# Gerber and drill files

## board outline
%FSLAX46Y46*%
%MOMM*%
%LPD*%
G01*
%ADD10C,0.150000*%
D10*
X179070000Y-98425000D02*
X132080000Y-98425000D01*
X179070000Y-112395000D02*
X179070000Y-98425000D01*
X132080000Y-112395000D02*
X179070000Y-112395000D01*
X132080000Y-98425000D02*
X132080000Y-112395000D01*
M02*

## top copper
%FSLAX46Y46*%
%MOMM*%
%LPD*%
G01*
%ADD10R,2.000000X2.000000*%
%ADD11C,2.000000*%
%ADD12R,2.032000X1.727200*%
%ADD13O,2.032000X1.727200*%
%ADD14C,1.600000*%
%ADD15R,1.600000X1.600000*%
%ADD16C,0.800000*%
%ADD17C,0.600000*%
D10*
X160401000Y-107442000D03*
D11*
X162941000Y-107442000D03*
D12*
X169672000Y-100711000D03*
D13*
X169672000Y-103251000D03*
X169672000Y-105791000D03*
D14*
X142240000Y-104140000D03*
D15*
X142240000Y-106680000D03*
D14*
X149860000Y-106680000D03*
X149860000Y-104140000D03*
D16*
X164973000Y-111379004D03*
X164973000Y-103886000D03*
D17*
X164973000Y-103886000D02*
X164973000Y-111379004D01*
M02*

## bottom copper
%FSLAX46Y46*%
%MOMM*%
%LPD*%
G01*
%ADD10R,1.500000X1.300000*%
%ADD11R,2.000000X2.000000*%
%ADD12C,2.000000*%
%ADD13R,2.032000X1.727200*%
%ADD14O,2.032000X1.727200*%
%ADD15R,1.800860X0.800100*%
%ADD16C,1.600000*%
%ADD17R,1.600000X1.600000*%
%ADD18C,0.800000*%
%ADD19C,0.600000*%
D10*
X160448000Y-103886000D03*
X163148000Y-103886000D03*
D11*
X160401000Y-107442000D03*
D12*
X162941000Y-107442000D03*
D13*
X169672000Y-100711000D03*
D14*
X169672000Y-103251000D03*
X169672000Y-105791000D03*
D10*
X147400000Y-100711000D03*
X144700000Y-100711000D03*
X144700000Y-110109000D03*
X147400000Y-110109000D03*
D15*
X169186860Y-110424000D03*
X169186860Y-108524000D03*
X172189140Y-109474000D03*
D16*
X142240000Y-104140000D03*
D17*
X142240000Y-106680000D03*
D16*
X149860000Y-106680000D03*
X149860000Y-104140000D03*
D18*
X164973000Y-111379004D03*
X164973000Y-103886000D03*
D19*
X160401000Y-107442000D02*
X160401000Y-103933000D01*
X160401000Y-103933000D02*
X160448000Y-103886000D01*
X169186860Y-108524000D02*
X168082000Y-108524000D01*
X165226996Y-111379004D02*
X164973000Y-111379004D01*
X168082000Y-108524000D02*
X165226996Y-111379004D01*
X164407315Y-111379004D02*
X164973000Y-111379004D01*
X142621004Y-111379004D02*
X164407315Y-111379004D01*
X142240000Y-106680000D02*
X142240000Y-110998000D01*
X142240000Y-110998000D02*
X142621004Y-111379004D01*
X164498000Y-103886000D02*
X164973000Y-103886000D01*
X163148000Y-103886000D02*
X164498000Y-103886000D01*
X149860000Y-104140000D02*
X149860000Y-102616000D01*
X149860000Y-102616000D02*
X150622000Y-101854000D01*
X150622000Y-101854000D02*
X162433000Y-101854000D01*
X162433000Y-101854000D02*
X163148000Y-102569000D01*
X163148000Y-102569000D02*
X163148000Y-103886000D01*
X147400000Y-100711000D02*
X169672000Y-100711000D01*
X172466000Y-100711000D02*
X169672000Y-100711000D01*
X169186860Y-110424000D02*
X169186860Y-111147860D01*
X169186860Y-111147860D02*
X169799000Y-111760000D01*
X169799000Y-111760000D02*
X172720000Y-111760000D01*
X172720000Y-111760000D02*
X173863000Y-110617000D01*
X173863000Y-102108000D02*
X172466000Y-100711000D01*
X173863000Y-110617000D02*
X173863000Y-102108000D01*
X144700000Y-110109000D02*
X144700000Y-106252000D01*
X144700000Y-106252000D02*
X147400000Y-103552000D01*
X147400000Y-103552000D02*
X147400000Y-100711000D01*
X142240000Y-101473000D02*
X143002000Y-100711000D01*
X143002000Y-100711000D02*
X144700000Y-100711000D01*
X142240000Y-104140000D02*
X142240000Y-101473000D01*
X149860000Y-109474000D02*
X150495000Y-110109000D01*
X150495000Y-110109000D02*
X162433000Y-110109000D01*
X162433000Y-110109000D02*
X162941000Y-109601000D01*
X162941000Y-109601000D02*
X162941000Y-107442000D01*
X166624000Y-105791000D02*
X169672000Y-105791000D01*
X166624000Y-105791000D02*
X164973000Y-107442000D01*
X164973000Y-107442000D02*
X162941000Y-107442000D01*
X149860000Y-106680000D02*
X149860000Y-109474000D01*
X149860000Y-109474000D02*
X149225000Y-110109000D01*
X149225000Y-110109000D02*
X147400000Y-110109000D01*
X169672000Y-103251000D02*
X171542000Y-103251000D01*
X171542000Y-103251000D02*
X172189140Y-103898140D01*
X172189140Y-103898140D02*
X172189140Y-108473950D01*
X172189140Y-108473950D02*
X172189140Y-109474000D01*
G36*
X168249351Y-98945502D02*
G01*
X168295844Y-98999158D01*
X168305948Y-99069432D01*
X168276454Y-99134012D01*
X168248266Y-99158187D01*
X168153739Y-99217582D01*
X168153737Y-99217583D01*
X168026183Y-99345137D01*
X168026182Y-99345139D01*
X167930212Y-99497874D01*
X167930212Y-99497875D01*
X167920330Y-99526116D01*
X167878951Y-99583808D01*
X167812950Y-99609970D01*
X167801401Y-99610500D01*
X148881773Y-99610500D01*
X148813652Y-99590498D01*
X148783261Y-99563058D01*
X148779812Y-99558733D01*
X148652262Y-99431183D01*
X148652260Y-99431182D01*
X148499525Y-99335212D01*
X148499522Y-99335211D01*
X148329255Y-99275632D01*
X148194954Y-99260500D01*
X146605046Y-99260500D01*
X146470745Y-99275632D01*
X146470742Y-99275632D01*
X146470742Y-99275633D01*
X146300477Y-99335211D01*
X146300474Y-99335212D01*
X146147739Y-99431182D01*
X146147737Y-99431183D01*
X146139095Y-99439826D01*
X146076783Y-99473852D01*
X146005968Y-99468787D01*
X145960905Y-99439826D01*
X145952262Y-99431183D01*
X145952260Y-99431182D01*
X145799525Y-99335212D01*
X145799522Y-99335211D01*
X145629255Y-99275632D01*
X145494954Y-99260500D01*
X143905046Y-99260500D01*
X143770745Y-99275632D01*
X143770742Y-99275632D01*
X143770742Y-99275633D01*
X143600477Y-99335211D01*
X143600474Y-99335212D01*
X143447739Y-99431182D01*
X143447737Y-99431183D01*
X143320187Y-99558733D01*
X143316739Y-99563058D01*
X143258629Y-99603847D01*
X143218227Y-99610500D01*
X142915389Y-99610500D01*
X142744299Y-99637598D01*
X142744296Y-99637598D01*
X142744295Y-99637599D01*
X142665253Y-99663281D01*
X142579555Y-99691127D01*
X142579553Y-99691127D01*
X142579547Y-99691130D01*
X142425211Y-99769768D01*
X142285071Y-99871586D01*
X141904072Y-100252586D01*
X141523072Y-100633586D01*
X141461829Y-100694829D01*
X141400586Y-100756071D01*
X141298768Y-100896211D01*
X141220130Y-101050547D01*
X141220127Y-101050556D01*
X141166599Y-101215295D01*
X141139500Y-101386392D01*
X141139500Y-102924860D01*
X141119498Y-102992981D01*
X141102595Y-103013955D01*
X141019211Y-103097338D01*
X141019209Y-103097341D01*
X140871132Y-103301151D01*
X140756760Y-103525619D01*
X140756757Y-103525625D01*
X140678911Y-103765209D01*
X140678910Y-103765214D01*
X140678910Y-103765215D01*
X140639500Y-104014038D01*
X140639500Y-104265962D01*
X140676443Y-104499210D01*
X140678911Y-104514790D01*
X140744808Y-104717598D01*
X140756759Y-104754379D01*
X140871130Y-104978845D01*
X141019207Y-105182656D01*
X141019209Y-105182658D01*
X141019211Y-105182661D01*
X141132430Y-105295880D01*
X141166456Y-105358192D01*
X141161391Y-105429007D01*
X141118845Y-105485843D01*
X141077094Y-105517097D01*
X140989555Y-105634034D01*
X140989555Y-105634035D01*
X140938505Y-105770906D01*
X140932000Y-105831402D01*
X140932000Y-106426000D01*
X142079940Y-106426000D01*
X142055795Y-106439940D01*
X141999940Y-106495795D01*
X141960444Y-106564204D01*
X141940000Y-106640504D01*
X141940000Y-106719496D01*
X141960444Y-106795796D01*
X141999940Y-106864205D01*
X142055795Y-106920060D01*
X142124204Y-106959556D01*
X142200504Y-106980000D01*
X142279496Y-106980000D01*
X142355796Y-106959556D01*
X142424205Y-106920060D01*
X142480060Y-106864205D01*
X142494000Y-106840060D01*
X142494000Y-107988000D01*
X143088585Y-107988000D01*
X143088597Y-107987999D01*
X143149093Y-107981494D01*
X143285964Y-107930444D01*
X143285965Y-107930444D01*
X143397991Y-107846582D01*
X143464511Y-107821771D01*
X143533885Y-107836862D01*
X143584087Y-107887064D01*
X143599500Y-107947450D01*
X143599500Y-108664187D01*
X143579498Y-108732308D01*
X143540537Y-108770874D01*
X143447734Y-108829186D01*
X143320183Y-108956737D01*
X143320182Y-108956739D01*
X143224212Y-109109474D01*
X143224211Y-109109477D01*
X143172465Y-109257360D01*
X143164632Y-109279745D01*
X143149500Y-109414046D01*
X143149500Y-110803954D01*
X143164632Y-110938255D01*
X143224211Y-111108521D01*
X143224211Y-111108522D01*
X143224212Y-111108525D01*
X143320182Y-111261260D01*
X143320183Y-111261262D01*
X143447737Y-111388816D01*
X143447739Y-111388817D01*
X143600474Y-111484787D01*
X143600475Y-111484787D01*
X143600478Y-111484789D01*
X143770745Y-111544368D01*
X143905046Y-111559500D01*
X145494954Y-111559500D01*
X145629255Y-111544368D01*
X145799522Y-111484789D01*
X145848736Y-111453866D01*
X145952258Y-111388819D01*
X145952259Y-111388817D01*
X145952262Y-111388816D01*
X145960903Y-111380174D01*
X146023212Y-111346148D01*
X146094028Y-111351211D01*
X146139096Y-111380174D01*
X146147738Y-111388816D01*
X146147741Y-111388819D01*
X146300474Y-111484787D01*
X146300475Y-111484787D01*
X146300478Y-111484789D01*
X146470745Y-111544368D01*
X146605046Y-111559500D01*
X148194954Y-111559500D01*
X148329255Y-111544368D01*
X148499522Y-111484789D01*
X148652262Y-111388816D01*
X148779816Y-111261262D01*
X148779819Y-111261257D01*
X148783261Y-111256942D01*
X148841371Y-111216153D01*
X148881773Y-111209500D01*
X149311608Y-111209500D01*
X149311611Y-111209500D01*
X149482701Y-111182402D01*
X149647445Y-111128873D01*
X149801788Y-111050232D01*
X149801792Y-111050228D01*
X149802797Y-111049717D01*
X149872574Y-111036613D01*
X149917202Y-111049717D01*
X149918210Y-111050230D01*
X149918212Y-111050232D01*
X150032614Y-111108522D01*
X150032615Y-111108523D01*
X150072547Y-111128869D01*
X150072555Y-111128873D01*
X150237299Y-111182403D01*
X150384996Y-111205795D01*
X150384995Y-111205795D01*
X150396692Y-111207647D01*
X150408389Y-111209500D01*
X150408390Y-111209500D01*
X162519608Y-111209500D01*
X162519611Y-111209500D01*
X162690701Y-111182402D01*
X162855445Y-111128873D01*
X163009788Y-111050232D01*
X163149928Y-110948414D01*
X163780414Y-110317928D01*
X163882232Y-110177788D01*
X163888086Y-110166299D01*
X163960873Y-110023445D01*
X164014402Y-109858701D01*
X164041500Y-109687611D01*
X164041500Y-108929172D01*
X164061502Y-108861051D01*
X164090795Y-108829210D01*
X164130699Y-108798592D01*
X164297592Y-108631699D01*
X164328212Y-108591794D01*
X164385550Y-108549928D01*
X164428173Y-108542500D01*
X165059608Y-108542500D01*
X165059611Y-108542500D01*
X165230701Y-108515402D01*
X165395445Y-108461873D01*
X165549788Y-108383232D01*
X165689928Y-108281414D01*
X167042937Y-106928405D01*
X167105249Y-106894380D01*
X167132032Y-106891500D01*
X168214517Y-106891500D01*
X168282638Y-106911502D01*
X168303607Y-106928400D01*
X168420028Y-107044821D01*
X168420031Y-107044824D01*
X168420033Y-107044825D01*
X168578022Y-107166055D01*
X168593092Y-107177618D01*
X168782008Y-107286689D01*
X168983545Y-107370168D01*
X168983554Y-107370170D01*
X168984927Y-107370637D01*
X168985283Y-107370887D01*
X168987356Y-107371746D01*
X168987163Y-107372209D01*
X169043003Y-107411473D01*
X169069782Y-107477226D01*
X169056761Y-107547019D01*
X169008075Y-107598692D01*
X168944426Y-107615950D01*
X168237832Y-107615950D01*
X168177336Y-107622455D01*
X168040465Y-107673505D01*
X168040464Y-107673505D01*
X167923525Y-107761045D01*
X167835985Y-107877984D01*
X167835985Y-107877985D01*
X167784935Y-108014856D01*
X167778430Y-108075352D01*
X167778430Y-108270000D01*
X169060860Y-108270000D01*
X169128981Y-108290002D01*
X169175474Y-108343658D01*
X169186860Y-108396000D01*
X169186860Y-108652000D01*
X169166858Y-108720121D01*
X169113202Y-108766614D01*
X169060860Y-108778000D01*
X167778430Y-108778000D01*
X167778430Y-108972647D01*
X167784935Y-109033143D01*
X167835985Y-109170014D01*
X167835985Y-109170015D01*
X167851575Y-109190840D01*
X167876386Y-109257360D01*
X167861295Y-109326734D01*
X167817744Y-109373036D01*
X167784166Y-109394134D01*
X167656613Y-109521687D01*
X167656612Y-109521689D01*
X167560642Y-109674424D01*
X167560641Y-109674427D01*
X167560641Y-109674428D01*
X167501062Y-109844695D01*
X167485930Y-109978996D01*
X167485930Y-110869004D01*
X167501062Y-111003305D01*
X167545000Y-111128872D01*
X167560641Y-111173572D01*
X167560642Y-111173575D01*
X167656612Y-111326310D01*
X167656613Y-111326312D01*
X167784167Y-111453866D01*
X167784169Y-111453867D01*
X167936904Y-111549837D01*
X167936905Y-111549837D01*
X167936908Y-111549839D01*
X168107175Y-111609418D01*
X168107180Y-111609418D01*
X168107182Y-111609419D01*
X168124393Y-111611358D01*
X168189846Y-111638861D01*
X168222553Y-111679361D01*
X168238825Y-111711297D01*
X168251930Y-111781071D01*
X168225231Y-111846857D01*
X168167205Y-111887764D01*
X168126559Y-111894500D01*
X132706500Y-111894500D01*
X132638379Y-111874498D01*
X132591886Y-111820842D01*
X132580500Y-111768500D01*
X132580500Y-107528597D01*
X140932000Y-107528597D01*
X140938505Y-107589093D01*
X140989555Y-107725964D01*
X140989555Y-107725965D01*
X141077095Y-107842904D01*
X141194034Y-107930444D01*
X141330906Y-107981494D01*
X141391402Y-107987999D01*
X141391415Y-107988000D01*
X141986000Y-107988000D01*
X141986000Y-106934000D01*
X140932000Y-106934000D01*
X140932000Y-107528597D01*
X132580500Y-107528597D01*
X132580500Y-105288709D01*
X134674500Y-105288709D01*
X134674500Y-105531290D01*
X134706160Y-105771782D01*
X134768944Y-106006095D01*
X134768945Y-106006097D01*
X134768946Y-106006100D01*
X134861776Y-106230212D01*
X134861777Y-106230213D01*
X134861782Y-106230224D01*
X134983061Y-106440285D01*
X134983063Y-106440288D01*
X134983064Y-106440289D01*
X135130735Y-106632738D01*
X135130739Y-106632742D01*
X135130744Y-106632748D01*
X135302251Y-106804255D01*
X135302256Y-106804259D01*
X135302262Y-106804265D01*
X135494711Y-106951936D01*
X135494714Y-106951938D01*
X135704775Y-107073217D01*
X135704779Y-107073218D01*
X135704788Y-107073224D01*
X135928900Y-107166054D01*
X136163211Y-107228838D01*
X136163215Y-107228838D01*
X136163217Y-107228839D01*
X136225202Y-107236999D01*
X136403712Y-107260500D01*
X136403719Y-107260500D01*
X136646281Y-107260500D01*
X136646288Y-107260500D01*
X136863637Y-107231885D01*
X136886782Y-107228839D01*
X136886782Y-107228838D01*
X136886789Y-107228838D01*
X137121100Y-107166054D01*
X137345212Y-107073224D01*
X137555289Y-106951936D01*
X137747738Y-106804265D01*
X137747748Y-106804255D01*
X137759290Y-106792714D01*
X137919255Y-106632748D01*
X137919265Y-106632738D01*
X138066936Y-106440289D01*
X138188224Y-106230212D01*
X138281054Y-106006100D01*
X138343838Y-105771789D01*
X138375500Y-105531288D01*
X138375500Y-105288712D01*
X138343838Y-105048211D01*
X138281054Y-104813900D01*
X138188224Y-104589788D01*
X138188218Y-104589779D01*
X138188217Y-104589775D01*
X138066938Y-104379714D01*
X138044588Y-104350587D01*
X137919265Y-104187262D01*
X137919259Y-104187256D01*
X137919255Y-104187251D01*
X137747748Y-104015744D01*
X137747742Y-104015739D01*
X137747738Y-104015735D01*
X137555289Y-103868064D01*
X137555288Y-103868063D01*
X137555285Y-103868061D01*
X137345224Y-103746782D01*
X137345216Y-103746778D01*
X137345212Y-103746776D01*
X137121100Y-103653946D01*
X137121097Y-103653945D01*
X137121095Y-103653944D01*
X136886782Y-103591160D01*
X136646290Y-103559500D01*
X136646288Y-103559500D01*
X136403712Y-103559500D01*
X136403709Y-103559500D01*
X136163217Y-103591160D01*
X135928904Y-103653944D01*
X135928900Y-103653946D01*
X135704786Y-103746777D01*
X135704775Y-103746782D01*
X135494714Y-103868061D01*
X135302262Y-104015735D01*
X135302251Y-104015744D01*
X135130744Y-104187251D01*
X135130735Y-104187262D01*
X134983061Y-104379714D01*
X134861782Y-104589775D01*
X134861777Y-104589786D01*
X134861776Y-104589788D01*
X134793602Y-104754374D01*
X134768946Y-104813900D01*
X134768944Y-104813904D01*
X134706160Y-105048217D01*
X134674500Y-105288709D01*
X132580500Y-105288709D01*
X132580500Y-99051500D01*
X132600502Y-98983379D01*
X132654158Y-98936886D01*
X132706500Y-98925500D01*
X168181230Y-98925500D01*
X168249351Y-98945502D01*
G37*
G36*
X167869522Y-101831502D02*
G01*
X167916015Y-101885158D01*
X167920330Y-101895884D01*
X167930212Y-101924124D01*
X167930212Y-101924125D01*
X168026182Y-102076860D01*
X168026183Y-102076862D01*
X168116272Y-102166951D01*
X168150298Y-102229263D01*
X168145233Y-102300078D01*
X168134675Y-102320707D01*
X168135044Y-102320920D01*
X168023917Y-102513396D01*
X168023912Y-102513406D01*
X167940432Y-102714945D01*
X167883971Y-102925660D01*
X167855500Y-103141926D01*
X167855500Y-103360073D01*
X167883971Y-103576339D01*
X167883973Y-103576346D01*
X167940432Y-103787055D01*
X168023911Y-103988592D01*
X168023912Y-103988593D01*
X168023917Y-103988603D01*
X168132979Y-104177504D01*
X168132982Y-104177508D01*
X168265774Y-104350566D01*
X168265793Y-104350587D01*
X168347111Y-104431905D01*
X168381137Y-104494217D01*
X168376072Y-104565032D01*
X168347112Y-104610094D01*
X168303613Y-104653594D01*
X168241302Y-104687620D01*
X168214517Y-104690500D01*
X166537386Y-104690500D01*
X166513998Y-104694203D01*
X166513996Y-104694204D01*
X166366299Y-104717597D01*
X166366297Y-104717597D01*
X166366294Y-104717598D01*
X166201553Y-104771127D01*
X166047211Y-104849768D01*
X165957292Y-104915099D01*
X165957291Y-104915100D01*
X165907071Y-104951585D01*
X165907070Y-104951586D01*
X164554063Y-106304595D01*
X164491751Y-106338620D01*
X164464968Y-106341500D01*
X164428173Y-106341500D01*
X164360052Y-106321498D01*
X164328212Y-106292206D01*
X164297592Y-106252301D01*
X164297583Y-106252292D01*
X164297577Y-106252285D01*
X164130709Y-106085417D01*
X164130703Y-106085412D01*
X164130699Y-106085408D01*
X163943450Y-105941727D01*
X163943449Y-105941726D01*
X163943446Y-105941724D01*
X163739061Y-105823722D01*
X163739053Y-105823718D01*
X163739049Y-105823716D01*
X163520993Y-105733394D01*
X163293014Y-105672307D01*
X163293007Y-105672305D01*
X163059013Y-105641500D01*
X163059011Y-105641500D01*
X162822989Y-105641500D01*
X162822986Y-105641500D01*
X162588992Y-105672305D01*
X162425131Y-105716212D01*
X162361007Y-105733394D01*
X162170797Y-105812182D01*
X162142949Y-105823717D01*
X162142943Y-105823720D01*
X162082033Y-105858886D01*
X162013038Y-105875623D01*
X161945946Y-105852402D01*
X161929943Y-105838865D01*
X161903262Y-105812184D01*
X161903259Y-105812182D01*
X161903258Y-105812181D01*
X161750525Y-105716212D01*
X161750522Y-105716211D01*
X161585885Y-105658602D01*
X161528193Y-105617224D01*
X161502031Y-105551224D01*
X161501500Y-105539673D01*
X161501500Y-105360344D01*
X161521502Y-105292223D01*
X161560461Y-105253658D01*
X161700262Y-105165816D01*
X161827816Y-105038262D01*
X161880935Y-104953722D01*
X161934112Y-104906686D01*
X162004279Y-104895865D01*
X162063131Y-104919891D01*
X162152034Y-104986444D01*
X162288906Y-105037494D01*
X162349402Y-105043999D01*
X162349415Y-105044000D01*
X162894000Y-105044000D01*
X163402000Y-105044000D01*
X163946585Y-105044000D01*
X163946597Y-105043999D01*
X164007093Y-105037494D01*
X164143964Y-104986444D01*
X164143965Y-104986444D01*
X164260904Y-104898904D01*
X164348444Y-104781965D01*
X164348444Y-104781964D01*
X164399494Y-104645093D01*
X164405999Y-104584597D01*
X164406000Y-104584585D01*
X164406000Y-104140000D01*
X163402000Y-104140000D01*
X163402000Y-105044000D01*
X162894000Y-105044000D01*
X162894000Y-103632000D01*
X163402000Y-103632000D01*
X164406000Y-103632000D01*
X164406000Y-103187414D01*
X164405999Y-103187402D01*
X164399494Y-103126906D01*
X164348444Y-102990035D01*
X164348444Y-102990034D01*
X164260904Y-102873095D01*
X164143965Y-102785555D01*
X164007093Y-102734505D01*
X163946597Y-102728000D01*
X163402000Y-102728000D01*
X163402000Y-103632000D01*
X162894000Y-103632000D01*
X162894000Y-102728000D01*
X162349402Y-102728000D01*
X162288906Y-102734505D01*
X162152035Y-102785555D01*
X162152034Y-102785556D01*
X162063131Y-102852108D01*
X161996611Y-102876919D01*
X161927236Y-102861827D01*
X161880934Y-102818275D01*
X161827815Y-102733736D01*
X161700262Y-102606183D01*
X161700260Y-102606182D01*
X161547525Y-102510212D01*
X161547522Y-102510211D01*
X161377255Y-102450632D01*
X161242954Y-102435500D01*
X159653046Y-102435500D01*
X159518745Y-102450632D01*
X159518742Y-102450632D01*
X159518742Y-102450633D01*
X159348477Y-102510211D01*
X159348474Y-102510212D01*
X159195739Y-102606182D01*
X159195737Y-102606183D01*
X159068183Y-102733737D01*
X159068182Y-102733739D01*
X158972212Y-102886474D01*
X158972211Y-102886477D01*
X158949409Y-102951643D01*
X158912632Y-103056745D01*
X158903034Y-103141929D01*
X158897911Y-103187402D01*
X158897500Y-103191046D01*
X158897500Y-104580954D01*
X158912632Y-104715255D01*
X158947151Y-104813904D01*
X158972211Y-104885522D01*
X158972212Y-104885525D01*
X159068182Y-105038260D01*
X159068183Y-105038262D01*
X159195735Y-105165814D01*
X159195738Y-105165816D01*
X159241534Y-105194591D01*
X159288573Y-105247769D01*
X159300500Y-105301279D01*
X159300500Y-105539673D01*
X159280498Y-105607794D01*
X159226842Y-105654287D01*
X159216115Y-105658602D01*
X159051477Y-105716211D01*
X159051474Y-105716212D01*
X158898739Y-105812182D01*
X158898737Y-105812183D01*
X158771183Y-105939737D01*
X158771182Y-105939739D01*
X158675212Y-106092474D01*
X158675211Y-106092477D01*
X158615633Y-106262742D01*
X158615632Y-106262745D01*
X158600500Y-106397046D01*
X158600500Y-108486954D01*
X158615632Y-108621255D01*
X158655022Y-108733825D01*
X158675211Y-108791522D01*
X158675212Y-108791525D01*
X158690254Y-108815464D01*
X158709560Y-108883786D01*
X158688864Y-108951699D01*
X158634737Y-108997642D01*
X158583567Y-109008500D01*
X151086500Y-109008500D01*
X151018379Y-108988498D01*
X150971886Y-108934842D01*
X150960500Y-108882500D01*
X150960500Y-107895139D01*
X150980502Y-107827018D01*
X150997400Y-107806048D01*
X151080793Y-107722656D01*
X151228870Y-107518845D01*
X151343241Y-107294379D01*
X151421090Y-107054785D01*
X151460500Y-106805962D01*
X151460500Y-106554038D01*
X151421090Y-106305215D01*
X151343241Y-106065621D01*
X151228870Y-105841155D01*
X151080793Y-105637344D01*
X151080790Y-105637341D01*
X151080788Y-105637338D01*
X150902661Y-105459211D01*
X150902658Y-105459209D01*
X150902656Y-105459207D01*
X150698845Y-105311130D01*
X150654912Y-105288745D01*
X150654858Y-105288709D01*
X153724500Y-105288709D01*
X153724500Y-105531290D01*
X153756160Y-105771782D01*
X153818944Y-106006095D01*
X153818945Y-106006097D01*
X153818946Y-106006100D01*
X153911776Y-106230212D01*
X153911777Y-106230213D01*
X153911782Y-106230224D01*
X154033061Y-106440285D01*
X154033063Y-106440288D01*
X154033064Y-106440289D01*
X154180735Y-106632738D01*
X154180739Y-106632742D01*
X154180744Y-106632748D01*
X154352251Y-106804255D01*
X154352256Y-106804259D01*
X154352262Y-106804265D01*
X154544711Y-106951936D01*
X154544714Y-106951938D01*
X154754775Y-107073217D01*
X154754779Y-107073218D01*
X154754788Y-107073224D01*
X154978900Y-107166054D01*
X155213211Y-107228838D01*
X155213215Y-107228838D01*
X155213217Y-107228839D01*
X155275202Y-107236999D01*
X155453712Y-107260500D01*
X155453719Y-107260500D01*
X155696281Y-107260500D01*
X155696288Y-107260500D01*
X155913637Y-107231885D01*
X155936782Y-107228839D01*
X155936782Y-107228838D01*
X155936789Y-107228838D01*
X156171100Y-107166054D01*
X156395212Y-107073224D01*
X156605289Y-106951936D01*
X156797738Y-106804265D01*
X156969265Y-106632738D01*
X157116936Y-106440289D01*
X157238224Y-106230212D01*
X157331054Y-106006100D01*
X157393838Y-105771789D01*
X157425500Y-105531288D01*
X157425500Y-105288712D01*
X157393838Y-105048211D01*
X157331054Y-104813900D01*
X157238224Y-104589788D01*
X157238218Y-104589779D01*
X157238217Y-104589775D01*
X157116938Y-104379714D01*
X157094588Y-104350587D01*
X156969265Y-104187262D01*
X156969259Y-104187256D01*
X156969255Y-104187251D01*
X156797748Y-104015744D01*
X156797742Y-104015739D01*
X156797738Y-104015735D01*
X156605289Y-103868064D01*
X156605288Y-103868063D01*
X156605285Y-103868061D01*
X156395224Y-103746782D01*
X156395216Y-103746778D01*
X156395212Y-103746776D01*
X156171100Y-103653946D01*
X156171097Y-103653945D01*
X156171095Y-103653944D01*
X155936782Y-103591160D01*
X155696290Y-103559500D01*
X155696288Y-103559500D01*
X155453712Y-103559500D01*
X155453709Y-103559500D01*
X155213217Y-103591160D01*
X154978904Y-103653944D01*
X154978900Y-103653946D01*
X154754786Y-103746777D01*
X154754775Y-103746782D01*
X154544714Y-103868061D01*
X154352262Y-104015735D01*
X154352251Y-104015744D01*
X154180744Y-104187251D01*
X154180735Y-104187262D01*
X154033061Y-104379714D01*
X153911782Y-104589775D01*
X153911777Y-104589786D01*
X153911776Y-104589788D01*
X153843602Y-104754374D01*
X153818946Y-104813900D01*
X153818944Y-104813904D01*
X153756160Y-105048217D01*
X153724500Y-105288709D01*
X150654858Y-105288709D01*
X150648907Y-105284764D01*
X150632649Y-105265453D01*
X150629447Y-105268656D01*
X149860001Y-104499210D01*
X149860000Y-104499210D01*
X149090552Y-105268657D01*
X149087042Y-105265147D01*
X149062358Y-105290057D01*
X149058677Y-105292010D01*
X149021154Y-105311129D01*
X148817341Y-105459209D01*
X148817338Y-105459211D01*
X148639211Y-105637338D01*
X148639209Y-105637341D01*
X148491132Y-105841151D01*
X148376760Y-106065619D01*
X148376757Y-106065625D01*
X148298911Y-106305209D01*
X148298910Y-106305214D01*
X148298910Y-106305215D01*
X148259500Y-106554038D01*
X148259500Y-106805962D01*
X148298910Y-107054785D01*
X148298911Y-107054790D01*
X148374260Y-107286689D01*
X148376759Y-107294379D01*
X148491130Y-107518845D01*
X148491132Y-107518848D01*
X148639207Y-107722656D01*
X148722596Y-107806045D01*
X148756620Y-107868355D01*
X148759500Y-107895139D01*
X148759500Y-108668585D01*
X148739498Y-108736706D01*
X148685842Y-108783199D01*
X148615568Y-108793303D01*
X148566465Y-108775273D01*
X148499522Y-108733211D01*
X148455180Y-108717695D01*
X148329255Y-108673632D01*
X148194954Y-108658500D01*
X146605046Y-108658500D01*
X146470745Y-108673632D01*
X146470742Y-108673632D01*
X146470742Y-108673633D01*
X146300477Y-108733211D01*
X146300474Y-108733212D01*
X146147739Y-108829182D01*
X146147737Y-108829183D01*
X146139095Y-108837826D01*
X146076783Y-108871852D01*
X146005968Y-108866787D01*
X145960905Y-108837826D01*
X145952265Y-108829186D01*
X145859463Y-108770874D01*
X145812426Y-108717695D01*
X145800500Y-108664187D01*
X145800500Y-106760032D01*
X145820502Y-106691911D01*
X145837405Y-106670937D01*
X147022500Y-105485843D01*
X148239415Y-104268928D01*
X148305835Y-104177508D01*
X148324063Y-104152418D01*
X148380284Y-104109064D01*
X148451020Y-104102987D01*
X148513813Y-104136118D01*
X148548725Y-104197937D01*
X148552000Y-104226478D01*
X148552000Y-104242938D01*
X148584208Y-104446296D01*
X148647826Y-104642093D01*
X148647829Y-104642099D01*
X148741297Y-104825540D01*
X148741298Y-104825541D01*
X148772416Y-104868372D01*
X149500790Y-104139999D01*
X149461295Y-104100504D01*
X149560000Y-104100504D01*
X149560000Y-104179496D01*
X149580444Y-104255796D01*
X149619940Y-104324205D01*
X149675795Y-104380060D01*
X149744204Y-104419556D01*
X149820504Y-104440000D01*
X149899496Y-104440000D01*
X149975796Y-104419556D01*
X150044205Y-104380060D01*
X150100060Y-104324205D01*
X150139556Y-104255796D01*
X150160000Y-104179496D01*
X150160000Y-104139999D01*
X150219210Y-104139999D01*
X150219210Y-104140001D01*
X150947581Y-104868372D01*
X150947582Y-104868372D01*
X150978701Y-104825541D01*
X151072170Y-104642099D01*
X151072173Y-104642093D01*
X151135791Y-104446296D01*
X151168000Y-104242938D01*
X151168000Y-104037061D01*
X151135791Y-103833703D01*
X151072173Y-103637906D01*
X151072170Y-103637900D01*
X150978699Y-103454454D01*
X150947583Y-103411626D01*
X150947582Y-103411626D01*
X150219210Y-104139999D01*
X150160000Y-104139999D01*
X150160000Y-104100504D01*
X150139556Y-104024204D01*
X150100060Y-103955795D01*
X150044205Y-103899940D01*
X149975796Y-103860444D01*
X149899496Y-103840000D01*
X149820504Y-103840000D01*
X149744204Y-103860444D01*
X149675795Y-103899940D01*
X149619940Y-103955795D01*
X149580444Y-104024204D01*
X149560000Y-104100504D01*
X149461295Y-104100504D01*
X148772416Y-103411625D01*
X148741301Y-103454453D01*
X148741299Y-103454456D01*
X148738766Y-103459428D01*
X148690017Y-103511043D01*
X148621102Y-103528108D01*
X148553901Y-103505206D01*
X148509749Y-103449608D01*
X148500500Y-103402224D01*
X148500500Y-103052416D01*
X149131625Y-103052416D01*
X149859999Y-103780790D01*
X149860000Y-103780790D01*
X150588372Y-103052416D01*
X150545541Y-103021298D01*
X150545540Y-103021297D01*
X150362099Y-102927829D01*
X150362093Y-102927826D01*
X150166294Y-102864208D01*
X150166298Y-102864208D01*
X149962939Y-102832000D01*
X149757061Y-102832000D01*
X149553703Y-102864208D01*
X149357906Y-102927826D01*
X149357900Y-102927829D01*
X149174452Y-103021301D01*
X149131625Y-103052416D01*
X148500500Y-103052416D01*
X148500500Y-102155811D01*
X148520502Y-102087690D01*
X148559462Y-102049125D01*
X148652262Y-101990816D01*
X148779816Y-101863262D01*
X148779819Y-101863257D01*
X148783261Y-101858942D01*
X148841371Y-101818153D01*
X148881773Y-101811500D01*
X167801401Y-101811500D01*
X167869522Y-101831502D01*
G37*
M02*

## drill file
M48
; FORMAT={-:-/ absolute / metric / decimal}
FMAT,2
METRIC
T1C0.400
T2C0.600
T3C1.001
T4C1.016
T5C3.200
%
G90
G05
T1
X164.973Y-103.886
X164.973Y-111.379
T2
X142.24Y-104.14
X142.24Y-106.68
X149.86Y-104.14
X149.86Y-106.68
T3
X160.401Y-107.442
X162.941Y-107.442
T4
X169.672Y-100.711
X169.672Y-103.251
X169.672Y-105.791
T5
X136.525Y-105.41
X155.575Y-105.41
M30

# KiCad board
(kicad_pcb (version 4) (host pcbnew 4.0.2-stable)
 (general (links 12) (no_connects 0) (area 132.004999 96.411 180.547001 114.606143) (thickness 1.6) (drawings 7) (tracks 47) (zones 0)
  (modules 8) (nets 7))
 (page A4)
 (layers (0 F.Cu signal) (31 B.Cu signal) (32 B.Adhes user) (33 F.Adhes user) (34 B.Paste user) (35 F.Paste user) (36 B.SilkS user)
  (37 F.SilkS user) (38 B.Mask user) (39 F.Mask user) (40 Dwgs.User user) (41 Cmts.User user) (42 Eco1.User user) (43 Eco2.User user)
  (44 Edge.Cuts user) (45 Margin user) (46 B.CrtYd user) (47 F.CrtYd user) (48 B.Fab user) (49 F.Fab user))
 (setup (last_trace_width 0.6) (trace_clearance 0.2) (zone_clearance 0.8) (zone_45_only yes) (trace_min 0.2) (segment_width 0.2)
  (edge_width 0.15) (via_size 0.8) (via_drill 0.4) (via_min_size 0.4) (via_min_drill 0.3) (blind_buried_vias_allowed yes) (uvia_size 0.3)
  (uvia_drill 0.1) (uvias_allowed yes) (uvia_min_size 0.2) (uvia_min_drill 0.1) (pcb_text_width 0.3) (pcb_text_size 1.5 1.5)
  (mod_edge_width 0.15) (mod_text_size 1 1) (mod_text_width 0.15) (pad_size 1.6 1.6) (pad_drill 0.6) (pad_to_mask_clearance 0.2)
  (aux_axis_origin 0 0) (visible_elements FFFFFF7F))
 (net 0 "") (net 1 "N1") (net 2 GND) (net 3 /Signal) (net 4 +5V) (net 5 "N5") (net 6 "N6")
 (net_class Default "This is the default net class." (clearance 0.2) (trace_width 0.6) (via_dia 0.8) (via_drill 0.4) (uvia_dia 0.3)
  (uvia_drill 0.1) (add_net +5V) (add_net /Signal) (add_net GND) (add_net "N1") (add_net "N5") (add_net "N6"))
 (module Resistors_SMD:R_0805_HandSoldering (layer B.Cu) (at 161.798 103.886)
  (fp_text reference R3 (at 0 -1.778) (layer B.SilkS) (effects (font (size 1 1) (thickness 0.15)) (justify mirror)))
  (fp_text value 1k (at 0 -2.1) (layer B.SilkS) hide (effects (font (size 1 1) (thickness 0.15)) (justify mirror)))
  (pad 1 smd rect (at -1.35 0) (size 1.5 1.3) (layers B.Cu B.Paste B.Mask) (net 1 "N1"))
  (pad 2 smd rect (at 1.35 0) (size 1.5 1.3) (layers B.Cu B.Paste B.Mask) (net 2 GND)))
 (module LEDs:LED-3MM (layer F.Cu) (at 160.401 107.442)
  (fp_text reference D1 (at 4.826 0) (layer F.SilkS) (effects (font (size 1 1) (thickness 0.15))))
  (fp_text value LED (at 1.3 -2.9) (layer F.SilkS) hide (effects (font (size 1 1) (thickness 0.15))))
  (pad 1 thru_hole rect (at 0 0 90) (size 2 2) (drill 1.00076) (layers *.Cu *.Mask F.SilkS) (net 1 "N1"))
  (pad 2 thru_hole circle (at 2.54 0) (size 2 2) (drill 1.00076) (layers *.Cu *.Mask F.SilkS) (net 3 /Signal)))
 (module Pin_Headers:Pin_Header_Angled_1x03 (layer F.Cu) (at 169.672 100.711)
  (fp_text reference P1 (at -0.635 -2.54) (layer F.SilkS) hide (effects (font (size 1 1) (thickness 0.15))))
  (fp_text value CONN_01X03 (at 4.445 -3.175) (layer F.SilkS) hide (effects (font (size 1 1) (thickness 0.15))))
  (pad 1 thru_hole rect (at 0 0) (size 2.032 1.7272) (drill 1.016) (layers *.Cu *.Mask F.SilkS) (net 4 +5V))
  (pad 2 thru_hole oval (at 0 2.54) (size 2.032 1.7272) (drill 1.016) (layers *.Cu *.Mask F.SilkS) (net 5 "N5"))
  (pad 3 thru_hole oval (at 0 5.08) (size 2.032 1.7272) (drill 1.016) (layers *.Cu *.Mask F.SilkS) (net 3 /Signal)))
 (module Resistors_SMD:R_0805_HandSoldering (layer B.Cu) (at 146.05 100.711 180)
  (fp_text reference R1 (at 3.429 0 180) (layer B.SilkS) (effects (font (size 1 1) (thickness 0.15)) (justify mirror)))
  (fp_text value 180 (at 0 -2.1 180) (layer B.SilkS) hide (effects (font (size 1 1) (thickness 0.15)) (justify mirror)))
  (pad 1 smd rect (at -1.35 0 180) (size 1.5 1.3) (layers B.Cu B.Paste B.Mask) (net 4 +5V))
  (pad 2 smd rect (at 1.35 0 180) (size 1.5 1.3) (layers B.Cu B.Paste B.Mask) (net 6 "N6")))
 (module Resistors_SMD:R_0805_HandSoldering (layer B.Cu) (at 146.05 110.109)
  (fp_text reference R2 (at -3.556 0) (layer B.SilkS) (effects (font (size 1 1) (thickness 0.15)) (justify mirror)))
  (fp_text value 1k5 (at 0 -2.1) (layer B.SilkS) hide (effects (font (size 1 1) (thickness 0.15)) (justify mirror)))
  (pad 1 smd rect (at -1.35 0) (size 1.5 1.3) (layers B.Cu B.Paste B.Mask) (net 4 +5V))
  (pad 2 smd rect (at 1.35 0) (size 1.5 1.3) (layers B.Cu B.Paste B.Mask) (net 3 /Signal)))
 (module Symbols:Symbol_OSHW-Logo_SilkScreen (layer B.Cu) (at 175.133 102.235 180)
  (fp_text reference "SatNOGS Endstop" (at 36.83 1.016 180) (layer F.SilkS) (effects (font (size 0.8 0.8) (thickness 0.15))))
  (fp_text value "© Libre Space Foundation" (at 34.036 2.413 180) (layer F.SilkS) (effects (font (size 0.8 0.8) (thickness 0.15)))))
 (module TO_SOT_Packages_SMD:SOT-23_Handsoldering (layer B.Cu) (at 170.688 109.474 90)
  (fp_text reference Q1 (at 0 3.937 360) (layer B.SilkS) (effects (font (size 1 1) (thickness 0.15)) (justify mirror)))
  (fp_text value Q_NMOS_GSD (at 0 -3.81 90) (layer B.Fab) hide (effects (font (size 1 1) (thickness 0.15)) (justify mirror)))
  (pad 1 smd rect (at -0.95 -1.50114 90) (size 0.8001 1.80086) (layers B.Cu B.Paste B.Mask) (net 4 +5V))
  (pad 2 smd rect (at 0.95 -1.50114 90) (size 0.8001 1.80086) (layers B.Cu B.Paste B.Mask) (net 2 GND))
  (pad 3 smd rect (at 0 1.50114 90) (size 0.8001 1.80086) (layers B.Cu B.Paste B.Mask) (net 5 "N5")))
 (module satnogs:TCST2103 (layer F.Cu) (at 146.05 105.41)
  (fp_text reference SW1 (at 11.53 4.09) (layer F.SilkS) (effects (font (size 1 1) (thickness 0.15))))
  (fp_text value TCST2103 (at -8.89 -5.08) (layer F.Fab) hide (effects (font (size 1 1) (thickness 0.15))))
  (pad 1 thru_hole circle (at -3.81 -1.27) (size 1.6 1.6) (drill 0.6) (layers *.Cu *.Mask F.SilkS) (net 6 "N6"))
  (pad 2 thru_hole rect (at -3.81 1.27) (size 1.6 1.6) (drill 0.6) (layers *.Cu *.Mask F.SilkS) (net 2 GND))
  (pad 3 thru_hole circle (at 3.81 1.27) (size 1.6 1.6) (drill 0.6) (layers *.Cu *.Mask F.SilkS) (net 3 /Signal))
  (pad 4 thru_hole circle (at 3.81 -1.27) (size 1.6 1.6) (drill 0.6) (layers *.Cu *.Mask F.SilkS) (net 2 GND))
  (pad "" np_thru_hole circle (at 9.525 0) (size 3.2 3.2) (drill 3.2) (layers *.Cu *.Mask F.SilkS))
  (pad "" np_thru_hole circle (at -9.525 0) (size 3.2 3.2) (drill 3.2) (layers *.Cu *.Mask F.SilkS)))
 (gr_line (start 179.07 98.425) (end 132.08 98.425) (angle 90) (layer Edge.Cuts) (width 0.15))
 (gr_line (start 179.07 112.395) (end 179.07 98.425) (angle 90) (layer Edge.Cuts) (width 0.15))
 (gr_line (start 132.08 112.395) (end 179.07 112.395) (angle 90) (layer Edge.Cuts) (width 0.15))
 (gr_line (start 132.08 98.425) (end 132.08 112.395) (angle 90) (layer Edge.Cuts) (width 0.15))
 (segment (start 160.401 107.442) (end 160.401 103.933) (width 0.6) (layer B.Cu) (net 1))
 (segment (start 160.401 103.933) (end 160.448 103.886) (width 0.6) (layer B.Cu) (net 1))
 (segment (start 169.18686 108.524) (end 168.082 108.524) (width 0.6) (layer B.Cu) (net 2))
 (segment (start 165.226996 111.379004) (end 164.973 111.379004) (width 0.6) (layer B.Cu) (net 2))
 (segment (start 168.082 108.524) (end 165.226996 111.379004) (width 0.6) (layer B.Cu) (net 2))
 (segment (start 164.407315 111.379004) (end 164.973 111.379004) (width 0.6) (layer B.Cu) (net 2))
 (segment (start 142.621004 111.379004) (end 164.407315 111.379004) (width 0.6) (layer B.Cu) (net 2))
 (segment (start 142.24 106.68) (end 142.24 110.998) (width 0.6) (layer B.Cu) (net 2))
 (via (at 164.973 111.379004) (size 0.8) (drill 0.4) (layers F.Cu B.Cu) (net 2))
 (segment (start 142.24 110.998) (end 142.621004 111.379004) (width 0.6) (layer B.Cu) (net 2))
 (segment (start 164.973 103.886) (end 164.973 111.379004) (width 0.6) (layer F.Cu) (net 2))
 (segment (start 164.498 103.886) (end 164.973 103.886) (width 0.6) (layer B.Cu) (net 2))
 (via (at 164.973 103.886) (size 0.8) (drill 0.4) (layers F.Cu B.Cu) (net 2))
 (segment (start 163.148 103.886) (end 164.498 103.886) (width 0.6) (layer B.Cu) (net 2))
 (segment (start 149.86 104.14) (end 149.86 102.616) (width 0.6) (layer B.Cu) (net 2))
 (segment (start 149.86 102.616) (end 150.622 101.854) (width 0.6) (layer B.Cu) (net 2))
 (segment (start 150.622 101.854) (end 162.433 101.854) (width 0.6) (layer B.Cu) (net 2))
 (segment (start 162.433 101.854) (end 163.148 102.569) (width 0.6) (layer B.Cu) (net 2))
 (segment (start 163.148 102.569) (end 163.148 103.886) (width 0.6) (layer B.Cu) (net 2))
 (segment (start 147.4 100.711) (end 169.672 100.711) (width 0.6) (layer B.Cu) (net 4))
 (segment (start 172.466 100.711) (end 169.672 100.711) (width 0.6) (layer B.Cu) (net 4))
 (segment (start 169.18686 110.424) (end 169.18686 111.14786) (width 0.6) (layer B.Cu) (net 4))
 (segment (start 169.18686 111.14786) (end 169.799 111.76) (width 0.6) (layer B.Cu) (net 4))
 (segment (start 169.799 111.76) (end 172.72 111.76) (width 0.6) (layer B.Cu) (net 4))
 (segment (start 172.72 111.76) (end 173.863 110.617) (width 0.6) (layer B.Cu) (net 4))
 (segment (start 173.863 102.108) (end 172.466 100.711) (width 0.6) (layer B.Cu) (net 4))
 (segment (start 173.863 110.617) (end 173.863 102.108) (width 0.6) (layer B.Cu) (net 4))
 (segment (start 144.7 110.109) (end 144.7 106.252) (width 0.6) (layer B.Cu) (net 4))
 (segment (start 144.7 106.252) (end 147.4 103.552) (width 0.6) (layer B.Cu) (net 4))
 (segment (start 147.4 103.552) (end 147.4 100.711) (width 0.6) (layer B.Cu) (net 4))
 (segment (start 142.24 101.473) (end 143.002 100.711) (width 0.6) (layer B.Cu) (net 6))
 (segment (start 143.002 100.711) (end 144.7 100.711) (width 0.6) (layer B.Cu) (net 6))
 (segment (start 142.24 104.14) (end 142.24 101.473) (width 0.6) (layer B.Cu) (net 6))
 (segment (start 149.86 109.474) (end 150.495 110.109) (width 0.6) (layer B.Cu) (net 3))
 (segment (start 150.495 110.109) (end 162.433 110.109) (width 0.6) (layer B.Cu) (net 3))
 (segment (start 162.433 110.109) (end 162.941 109.601) (width 0.6) (layer B.Cu) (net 3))
 (segment (start 162.941 109.601) (end 162.941 107.442) (width 0.6) (layer B.Cu) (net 3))
 (segment (start 166.624 105.791) (end 169.672 105.791) (width 0.6) (layer B.Cu) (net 3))
 (segment (start 166.624 105.791) (end 164.973 107.442) (width 0.6) (layer B.Cu) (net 3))
 (segment (start 164.973 107.442) (end 162.941 107.442) (width 0.6) (layer B.Cu) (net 3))
 (segment (start 149.86 106.68) (end 149.86 109.474) (width 0.6) (layer B.Cu) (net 3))
 (segment (start 149.86 109.474) (end 149.225 110.109) (width 0.6) (layer B.Cu) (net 3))
 (segment (start 149.225 110.109) (end 147.4 110.109) (width 0.6) (layer B.Cu) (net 3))
 (segment (start 169.672 103.251) (end 171.542 103.251) (width 0.6) (layer B.Cu) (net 5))
 (segment (start 171.542 103.251) (end 172.18914 103.89814) (width 0.6) (layer B.Cu) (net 5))
 (segment (start 172.18914 103.89814) (end 172.18914 108.47395) (width 0.6) (layer B.Cu) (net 5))
 (segment (start 172.18914 108.47395) (end 172.18914 109.474) (width 0.6) (layer B.Cu) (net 5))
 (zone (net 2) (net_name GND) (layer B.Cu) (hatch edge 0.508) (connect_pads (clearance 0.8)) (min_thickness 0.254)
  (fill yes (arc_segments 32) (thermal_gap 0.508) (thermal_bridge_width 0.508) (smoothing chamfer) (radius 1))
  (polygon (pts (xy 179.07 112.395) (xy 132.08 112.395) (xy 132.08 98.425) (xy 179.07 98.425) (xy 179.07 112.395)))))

